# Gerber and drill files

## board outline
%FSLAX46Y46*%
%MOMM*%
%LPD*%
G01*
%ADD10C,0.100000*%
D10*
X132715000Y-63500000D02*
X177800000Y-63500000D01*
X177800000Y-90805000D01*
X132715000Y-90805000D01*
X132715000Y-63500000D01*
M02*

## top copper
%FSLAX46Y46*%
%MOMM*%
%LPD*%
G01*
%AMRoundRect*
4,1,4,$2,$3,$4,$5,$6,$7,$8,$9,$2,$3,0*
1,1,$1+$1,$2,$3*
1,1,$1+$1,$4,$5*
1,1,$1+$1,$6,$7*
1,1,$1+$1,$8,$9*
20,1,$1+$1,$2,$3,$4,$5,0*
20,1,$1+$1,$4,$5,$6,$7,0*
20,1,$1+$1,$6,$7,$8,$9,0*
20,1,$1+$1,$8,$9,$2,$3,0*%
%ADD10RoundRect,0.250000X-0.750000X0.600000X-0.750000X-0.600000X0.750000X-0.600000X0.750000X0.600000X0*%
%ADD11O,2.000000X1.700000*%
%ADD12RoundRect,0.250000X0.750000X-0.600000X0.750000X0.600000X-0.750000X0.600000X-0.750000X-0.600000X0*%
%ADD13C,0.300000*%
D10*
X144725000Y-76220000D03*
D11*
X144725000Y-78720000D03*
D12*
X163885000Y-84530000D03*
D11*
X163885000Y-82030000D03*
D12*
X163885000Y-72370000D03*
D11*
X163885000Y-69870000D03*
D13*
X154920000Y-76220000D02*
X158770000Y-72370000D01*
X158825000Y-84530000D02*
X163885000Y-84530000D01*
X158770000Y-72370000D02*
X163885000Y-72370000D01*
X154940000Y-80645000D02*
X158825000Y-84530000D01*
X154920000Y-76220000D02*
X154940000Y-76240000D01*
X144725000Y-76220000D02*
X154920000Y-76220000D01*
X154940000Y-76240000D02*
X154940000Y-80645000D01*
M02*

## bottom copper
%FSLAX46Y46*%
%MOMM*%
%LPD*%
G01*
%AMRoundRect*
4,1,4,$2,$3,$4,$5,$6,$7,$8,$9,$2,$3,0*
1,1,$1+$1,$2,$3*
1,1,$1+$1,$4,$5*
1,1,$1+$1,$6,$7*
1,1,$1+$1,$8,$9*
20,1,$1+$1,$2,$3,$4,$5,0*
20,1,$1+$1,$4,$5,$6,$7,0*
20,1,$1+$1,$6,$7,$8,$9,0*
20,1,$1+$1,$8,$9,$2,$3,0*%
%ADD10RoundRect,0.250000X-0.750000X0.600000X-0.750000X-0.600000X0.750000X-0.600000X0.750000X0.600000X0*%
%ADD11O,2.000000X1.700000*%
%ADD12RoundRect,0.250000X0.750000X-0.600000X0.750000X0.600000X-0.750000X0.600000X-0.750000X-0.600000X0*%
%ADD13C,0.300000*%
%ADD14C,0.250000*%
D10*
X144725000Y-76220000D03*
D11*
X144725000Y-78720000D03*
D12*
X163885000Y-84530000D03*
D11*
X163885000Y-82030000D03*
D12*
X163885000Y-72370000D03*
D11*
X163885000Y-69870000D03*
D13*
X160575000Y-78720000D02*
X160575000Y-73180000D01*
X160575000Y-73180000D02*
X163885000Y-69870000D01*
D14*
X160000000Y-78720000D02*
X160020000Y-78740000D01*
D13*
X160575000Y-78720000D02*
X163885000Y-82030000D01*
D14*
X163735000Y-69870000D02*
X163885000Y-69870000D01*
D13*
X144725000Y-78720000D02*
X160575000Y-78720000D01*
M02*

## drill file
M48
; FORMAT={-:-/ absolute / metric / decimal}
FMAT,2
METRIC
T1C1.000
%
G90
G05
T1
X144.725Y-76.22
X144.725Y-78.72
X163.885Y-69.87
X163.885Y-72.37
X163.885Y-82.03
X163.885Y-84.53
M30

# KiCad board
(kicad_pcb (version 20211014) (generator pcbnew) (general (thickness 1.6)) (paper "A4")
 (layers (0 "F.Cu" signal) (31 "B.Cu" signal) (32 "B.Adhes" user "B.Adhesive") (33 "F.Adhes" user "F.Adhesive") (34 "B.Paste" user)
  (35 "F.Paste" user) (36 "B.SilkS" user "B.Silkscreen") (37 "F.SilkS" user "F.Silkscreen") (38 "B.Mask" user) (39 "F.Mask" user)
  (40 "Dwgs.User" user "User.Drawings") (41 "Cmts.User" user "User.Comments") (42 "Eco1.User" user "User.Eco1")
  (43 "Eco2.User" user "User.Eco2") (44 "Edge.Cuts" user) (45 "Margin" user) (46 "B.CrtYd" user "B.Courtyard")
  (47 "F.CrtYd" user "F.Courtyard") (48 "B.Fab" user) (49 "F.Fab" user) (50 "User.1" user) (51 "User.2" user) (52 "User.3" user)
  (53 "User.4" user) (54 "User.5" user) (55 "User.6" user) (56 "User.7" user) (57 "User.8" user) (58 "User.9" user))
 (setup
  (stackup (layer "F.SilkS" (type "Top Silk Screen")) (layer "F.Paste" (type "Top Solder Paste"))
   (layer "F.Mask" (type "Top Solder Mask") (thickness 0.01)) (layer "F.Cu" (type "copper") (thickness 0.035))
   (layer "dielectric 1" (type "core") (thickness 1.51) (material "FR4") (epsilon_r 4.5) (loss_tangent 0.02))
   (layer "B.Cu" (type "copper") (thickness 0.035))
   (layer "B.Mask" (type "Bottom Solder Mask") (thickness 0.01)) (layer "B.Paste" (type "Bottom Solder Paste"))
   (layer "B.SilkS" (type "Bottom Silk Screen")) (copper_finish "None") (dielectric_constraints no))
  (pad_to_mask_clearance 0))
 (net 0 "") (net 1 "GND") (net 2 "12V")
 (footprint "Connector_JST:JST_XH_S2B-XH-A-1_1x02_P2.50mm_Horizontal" (layer "F.Cu") (at 144.725 76.22 -90)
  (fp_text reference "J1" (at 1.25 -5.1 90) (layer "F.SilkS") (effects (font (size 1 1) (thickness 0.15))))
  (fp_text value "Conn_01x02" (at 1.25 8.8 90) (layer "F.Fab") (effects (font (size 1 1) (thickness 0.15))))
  (pad "1" thru_hole roundrect (at 0 0 270) (size 1.7 2) (drill 1) (layers *.Cu *.Mask) (roundrect_rratio 0.147059) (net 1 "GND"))
  (pad "2" thru_hole oval (at 2.5 0 270) (size 1.7 2) (drill 1) (layers *.Cu *.Mask) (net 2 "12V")))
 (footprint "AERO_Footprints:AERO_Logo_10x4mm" (layer "F.Cu") (at 142.875 68.58)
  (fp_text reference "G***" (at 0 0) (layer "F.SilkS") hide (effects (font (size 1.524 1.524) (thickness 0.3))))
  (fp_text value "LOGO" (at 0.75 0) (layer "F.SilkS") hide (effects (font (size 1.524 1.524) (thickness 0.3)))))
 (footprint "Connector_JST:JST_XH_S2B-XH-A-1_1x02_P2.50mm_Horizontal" (layer "F.Cu") (at 163.885 84.53 90)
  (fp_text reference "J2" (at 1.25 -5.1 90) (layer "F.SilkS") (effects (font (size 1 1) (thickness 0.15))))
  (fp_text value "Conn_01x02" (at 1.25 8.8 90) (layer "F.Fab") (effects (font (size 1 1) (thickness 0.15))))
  (pad "1" thru_hole roundrect (at 0 0 90) (size 1.7 2) (drill 1) (layers *.Cu *.Mask) (roundrect_rratio 0.147059) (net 1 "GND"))
  (pad "2" thru_hole oval (at 2.5 0 90) (size 1.7 2) (drill 1) (layers *.Cu *.Mask) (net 2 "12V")))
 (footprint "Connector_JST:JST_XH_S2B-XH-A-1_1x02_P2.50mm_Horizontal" (layer "F.Cu") (at 163.885 72.37 90)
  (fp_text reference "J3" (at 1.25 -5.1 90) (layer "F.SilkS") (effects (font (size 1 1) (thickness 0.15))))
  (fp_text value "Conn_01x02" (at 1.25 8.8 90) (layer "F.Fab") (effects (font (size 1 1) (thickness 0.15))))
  (pad "1" thru_hole roundrect (at 0 0 90) (size 1.7 2) (drill 1) (layers *.Cu *.Mask) (roundrect_rratio 0.147059) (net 1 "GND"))
  (pad "2" thru_hole oval (at 2.5 0 90) (size 1.7 2) (drill 1) (layers *.Cu *.Mask) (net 2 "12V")))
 (gr_rect (start 132.715 63.5) (end 177.8 90.805) (layer "Edge.Cuts") (width 0.1) (fill none))
 (segment (start 154.92 76.22) (end 158.77 72.37) (width 0.3) (layer "F.Cu") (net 1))
 (segment (start 158.825 84.53) (end 163.885 84.53) (width 0.3) (layer "F.Cu") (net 1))
 (segment (start 158.77 72.37) (end 163.885 72.37) (width 0.3) (layer "F.Cu") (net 1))
 (segment (start 154.94 80.645) (end 158.825 84.53) (width 0.3) (layer "F.Cu") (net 1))
 (segment (start 154.92 76.22) (end 154.94 76.24) (width 0.3) (layer "F.Cu") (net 1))
 (segment (start 144.725 76.22) (end 154.92 76.22) (width 0.3) (layer "F.Cu") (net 1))
 (segment (start 154.94 76.24) (end 154.94 80.645) (width 0.3) (layer "F.Cu") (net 1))
 (segment (start 160.575 78.72) (end 160.575 73.18) (width 0.3) (layer "B.Cu") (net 2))
 (segment (start 160.575 73.18) (end 163.885 69.87) (width 0.3) (layer "B.Cu") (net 2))
 (segment (start 160 78.72) (end 160.02 78.74) (width 0.25) (layer "B.Cu") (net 2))
 (segment (start 160.575 78.72) (end 163.885 82.03) (width 0.3) (layer "B.Cu") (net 2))
 (segment (start 163.735 69.87) (end 163.885 69.87) (width 0.25) (layer "B.Cu") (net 2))
 (segment (start 144.725 78.72) (end 160.575 78.72) (width 0.3) (layer "B.Cu") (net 2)))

